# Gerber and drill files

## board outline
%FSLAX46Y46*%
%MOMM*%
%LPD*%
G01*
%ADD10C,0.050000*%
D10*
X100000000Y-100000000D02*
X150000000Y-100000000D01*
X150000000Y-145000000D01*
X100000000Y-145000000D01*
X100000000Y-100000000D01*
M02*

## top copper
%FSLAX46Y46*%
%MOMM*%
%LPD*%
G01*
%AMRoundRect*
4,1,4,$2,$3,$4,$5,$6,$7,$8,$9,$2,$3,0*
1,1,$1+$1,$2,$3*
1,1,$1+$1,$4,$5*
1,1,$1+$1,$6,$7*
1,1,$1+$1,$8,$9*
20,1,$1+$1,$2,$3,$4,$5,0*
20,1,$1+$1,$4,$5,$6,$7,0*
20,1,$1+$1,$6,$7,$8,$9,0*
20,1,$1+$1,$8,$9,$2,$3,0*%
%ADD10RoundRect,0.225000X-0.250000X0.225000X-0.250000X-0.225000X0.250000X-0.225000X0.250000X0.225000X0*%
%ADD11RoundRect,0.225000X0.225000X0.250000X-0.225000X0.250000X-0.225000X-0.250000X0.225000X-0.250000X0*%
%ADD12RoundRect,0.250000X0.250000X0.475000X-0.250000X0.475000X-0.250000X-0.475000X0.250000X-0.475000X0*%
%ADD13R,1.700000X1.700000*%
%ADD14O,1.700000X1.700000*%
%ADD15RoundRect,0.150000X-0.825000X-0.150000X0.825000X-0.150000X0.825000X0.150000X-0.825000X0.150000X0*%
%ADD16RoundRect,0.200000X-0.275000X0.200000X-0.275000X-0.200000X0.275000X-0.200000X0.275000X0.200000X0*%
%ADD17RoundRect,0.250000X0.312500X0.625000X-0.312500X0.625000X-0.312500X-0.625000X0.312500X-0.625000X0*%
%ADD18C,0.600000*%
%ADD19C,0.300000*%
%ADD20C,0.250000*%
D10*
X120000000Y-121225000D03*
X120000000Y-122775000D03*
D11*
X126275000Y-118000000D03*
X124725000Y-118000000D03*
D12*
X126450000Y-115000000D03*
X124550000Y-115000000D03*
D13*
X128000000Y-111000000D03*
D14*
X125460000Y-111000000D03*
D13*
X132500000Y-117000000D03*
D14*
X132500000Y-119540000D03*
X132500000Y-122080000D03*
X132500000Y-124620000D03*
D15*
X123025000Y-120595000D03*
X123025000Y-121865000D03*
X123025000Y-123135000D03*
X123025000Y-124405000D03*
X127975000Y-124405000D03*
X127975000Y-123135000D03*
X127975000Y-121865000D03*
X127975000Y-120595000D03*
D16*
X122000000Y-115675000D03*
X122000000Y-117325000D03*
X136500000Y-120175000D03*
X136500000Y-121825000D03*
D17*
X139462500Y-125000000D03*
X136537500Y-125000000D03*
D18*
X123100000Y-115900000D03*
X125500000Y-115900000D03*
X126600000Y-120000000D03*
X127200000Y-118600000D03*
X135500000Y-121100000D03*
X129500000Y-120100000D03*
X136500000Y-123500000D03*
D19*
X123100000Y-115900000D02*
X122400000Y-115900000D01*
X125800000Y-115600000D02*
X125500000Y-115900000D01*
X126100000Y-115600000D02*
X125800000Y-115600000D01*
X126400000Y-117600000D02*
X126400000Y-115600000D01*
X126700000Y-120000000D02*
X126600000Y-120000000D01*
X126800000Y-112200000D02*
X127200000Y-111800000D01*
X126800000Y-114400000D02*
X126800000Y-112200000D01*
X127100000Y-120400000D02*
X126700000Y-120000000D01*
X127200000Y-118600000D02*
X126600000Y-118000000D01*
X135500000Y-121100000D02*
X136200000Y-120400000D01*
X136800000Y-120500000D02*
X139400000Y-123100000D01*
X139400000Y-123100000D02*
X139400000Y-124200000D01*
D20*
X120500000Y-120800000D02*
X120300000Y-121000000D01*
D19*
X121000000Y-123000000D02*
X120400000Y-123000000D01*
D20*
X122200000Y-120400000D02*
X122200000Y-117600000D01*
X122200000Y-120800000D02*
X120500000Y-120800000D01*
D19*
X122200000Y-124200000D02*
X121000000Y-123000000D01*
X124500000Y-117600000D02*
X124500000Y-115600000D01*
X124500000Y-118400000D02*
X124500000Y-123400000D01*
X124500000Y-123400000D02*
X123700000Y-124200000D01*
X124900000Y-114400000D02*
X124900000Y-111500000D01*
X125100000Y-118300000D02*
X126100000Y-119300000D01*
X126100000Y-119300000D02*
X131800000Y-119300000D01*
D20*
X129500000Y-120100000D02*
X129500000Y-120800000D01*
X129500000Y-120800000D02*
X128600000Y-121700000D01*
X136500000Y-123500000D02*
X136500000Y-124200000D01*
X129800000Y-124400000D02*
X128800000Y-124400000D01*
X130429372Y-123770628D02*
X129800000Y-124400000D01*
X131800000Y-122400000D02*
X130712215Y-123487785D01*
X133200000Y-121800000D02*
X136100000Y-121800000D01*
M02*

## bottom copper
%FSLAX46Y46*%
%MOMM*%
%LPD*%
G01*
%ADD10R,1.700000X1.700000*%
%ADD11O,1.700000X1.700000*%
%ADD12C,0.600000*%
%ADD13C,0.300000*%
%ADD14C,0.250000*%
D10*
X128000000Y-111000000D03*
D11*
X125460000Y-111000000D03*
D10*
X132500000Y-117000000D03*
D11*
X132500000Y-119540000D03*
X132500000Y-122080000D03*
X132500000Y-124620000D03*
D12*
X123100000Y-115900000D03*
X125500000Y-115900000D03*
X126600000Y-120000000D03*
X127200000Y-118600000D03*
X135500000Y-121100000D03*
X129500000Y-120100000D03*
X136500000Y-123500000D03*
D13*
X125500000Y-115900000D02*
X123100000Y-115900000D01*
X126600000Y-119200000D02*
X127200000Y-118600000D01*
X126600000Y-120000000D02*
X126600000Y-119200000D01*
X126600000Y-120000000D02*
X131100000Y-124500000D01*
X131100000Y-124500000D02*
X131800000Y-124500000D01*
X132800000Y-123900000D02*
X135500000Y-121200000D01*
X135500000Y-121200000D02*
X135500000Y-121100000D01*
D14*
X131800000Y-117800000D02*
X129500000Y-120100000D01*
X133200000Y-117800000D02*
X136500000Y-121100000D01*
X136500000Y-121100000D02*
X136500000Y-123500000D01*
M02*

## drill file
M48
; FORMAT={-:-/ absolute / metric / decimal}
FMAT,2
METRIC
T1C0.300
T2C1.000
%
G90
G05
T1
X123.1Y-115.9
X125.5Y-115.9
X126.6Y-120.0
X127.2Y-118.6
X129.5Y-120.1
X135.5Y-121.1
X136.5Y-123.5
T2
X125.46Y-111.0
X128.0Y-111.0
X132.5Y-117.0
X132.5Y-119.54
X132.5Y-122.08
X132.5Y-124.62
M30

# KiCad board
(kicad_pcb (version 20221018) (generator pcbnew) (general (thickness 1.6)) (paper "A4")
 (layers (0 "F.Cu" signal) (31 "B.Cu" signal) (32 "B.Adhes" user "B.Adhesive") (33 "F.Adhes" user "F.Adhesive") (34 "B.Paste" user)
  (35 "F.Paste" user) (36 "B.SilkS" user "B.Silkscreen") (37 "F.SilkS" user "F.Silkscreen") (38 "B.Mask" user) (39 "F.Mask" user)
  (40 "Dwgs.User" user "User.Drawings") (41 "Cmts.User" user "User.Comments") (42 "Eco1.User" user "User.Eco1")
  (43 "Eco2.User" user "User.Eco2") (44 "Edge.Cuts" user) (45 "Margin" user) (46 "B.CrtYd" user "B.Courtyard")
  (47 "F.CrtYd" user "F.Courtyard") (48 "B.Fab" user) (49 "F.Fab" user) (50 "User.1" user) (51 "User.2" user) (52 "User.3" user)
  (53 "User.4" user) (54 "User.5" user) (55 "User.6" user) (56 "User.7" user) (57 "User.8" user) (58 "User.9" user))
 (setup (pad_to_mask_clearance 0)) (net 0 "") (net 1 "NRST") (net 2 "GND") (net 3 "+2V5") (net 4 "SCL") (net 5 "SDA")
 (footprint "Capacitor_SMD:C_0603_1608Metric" (layer "F.Cu") (at 120 122 -90)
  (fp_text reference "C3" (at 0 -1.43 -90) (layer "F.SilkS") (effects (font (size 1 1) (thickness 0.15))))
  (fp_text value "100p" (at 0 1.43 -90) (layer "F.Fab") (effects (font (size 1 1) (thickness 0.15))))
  (pad "1" smd roundrect (at -0.775 0 270) (size 0.9 0.95) (layers "F.Cu" "F.Paste" "F.Mask") (roundrect_rratio 0.25) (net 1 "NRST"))
  (pad "2" smd roundrect (at 0.775 0 270) (size 0.9 0.95) (layers "F.Cu" "F.Paste" "F.Mask") (roundrect_rratio 0.25) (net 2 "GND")))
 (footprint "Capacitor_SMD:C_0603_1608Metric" (layer "F.Cu") (at 125.5 118 180)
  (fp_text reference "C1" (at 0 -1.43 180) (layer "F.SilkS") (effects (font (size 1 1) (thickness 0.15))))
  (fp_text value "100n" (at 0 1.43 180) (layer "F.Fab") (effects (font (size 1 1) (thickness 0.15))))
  (pad "1" smd roundrect (at -0.775 0 180) (size 0.9 0.95) (layers "F.Cu" "F.Paste" "F.Mask") (roundrect_rratio 0.25) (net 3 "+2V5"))
  (pad "2" smd roundrect (at 0.775 0 180) (size 0.9 0.95) (layers "F.Cu" "F.Paste" "F.Mask") (roundrect_rratio 0.25) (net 2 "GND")))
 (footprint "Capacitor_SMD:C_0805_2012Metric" (layer "F.Cu") (at 125.5 115 180)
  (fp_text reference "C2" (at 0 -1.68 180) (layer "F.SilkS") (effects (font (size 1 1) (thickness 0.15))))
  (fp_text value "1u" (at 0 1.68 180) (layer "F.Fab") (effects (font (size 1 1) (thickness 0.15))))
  (pad "1" smd roundrect (at -0.95 0 180) (size 1 1.45) (layers "F.Cu" "F.Paste" "F.Mask") (roundrect_rratio 0.25) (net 3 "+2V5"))
  (pad "2" smd roundrect (at 0.95 0 180) (size 1 1.45) (layers "F.Cu" "F.Paste" "F.Mask") (roundrect_rratio 0.25) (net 2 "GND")))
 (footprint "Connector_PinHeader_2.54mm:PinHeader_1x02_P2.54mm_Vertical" (layer "F.Cu") (at 128 111 -90)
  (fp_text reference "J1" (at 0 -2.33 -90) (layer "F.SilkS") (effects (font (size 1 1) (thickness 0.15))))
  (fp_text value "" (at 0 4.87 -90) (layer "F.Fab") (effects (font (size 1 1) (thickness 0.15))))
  (pad "1" thru_hole rect (at 0 0 270) (size 1.7 1.7) (drill 1) (layers "*.Cu" "*.Mask") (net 3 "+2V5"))
  (pad "2" thru_hole oval (at 0 2.54 270) (size 1.7 1.7) (drill 1) (layers "*.Cu" "*.Mask") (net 2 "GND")))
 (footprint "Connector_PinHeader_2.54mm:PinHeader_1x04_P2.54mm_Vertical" (layer "F.Cu") (at 132.5 117)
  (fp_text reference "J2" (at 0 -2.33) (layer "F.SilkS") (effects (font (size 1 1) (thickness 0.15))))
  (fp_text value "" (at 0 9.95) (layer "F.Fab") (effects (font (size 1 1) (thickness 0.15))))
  (pad "1" thru_hole rect (at 0 0) (size 1.7 1.7) (drill 1) (layers "*.Cu" "*.Mask") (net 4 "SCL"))
  (pad "2" thru_hole oval (at 0 2.54) (size 1.7 1.7) (drill 1) (layers "*.Cu" "*.Mask") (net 2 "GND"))
  (pad "3" thru_hole oval (at 0 5.08) (size 1.7 1.7) (drill 1) (layers "*.Cu" "*.Mask") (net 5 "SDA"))
  (pad "4" thru_hole oval (at 0 7.62) (size 1.7 1.7) (drill 1) (layers "*.Cu" "*.Mask") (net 3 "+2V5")))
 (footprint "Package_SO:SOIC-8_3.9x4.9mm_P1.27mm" (layer "F.Cu") (at 125.5 122.5)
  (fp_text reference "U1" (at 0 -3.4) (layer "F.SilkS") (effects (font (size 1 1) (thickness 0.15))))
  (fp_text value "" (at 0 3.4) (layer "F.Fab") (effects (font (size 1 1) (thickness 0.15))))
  (pad "1" smd roundrect (at -2.475 -1.905) (size 1.95 0.6) (layers "F.Cu" "F.Paste" "F.Mask") (roundrect_rratio 0.25) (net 1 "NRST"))
  (pad "2" smd roundrect (at -2.475 -0.635) (size 1.95 0.6) (layers "F.Cu" "F.Paste" "F.Mask") (roundrect_rratio 0.25))
  (pad "3" smd roundrect (at -2.475 0.635) (size 1.95 0.6) (layers "F.Cu" "F.Paste" "F.Mask") (roundrect_rratio 0.25))
  (pad "4" smd roundrect (at -2.475 1.905) (size 1.95 0.6) (layers "F.Cu" "F.Paste" "F.Mask") (roundrect_rratio 0.25) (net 2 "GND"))
  (pad "5" smd roundrect (at 2.475 1.905) (size 1.95 0.6) (layers "F.Cu" "F.Paste" "F.Mask") (roundrect_rratio 0.25) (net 5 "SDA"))
  (pad "6" smd roundrect (at 2.475 0.635) (size 1.95 0.6) (layers "F.Cu" "F.Paste" "F.Mask") (roundrect_rratio 0.25))
  (pad "7" smd roundrect (at 2.475 -0.635) (size 1.95 0.6) (layers "F.Cu" "F.Paste" "F.Mask") (roundrect_rratio 0.25) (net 4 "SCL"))
  (pad "8" smd roundrect (at 2.475 -1.905) (size 1.95 0.6) (layers "F.Cu" "F.Paste" "F.Mask") (roundrect_rratio 0.25) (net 3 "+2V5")))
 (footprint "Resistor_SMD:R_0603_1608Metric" (layer "F.Cu") (at 122 116.5 -90)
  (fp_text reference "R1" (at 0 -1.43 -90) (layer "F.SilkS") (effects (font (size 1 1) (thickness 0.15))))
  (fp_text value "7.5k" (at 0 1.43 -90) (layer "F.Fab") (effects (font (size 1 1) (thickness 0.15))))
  (pad "1" smd roundrect (at -0.825 0 270) (size 0.8 0.95) (layers "F.Cu" "F.Paste" "F.Mask") (roundrect_rratio 0.25) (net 3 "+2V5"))
  (pad "2" smd roundrect (at 0.825 0 270) (size 0.8 0.95) (layers "F.Cu" "F.Paste" "F.Mask") (roundrect_rratio 0.25) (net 1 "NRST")))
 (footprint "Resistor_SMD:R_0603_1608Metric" (layer "F.Cu") (at 136.5 121 -90)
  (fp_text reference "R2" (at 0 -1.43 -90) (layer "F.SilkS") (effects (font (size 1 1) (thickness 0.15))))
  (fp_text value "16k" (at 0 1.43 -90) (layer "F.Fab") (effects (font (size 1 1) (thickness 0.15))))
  (pad "1" smd roundrect (at -0.825 0 270) (size 0.8 0.95) (layers "F.Cu" "F.Paste" "F.Mask") (roundrect_rratio 0.25) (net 3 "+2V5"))
  (pad "2" smd roundrect (at 0.825 0 270) (size 0.8 0.95) (layers "F.Cu" "F.Paste" "F.Mask") (roundrect_rratio 0.25) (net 5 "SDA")))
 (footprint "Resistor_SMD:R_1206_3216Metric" (layer "F.Cu") (at 138 125 180)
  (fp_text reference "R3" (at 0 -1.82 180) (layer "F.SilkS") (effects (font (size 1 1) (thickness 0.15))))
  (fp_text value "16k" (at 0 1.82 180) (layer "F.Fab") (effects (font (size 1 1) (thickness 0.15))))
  (pad "1" smd roundrect (at -1.4625 0 180) (size 1.125 1.75) (layers "F.Cu" "F.Paste" "F.Mask") (roundrect_rratio 0.222222) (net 3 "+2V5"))
  (pad "2" smd roundrect (at 1.4625 0 180) (size 1.125 1.75) (layers "F.Cu" "F.Paste" "F.Mask") (roundrect_rratio 0.222222) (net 4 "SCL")))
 (gr_rect (start 100 100) (end 150 145) (stroke (width 0.05) (type default)) (fill none) (layer "Edge.Cuts"))
 (segment (start 123.1 115.9) (end 122.4 115.9) (width 0.3) (layer "F.Cu") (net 3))
 (segment (start 125.8 115.6) (end 125.5 115.9) (width 0.3) (layer "F.Cu") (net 3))
 (segment (start 126.1 115.6) (end 125.8 115.6) (width 0.3) (layer "F.Cu") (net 3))
 (segment (start 126.4 117.6) (end 126.4 115.6) (width 0.3) (layer "F.Cu") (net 3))
 (segment (start 126.7 120) (end 126.6 120) (width 0.3) (layer "F.Cu") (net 3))
 (segment (start 126.8 112.2) (end 127.2 111.8) (width 0.3) (layer "F.Cu") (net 3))
 (segment (start 126.8 114.4) (end 126.8 112.2) (width 0.3) (layer "F.Cu") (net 3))
 (segment (start 127.1 120.4) (end 126.7 120) (width 0.3) (layer "F.Cu") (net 3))
 (segment (start 127.2 118.6) (end 126.6 118) (width 0.3) (layer "F.Cu") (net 3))
 (segment (start 135.5 121.1) (end 136.2 120.4) (width 0.3) (layer "F.Cu") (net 3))
 (segment (start 136.8 120.5) (end 139.4 123.1) (width 0.3) (layer "F.Cu") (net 3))
 (segment (start 139.4 123.1) (end 139.4 124.2) (width 0.3) (layer "F.Cu") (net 3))
 (via (at 123.1 115.9) (size 0.6) (drill 0.3) (layers "F.Cu" "B.Cu") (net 3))
 (via (at 125.5 115.9) (size 0.6) (drill 0.3) (layers "F.Cu" "B.Cu") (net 3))
 (via (at 126.6 120) (size 0.6) (drill 0.3) (layers "F.Cu" "B.Cu") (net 3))
 (via (at 127.2 118.6) (size 0.6) (drill 0.3) (layers "F.Cu" "B.Cu") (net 3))
 (via (at 135.5 121.1) (size 0.6) (drill 0.3) (layers "F.Cu" "B.Cu") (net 3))
 (segment (start 120.5 120.8) (end 120.3 121) (width 0.25) (layer "F.Cu") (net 1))
 (segment (start 121 123) (end 120.4 123) (width 0.3) (layer "F.Cu") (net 2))
 (segment (start 122.2 120.4) (end 122.2 117.6) (width 0.25) (layer "F.Cu") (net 1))
 (segment (start 122.2 120.8) (end 120.5 120.8) (width 0.25) (layer "F.Cu") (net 1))
 (segment (start 122.2 124.2) (end 121 123) (width 0.3) (layer "F.Cu") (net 2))
 (segment (start 124.5 117.6) (end 124.5 115.6) (width 0.3) (layer "F.Cu") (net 2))
 (segment (start 124.5 118.4) (end 124.5 123.4) (width 0.3) (layer "F.Cu") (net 2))
 (segment (start 124.5 123.4) (end 123.7 124.2) (width 0.3) (layer "F.Cu") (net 2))
 (segment (start 124.9 114.4) (end 124.9 111.5) (width 0.3) (layer "F.Cu") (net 2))
 (segment (start 125.1 118.3) (end 126.1 119.3) (width 0.3) (layer "F.Cu") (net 2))
 (segment (start 125.5 115.9) (end 123.1 115.9) (width 0.3) (layer "B.Cu") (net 3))
 (segment (start 126.1 119.3) (end 131.8 119.3) (width 0.3) (layer "F.Cu") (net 2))
 (segment (start 126.6 119.2) (end 127.2 118.6) (width 0.3) (layer "B.Cu") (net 3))
 (segment (start 126.6 120) (end 126.6 119.2) (width 0.3) (layer "B.Cu") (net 3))
 (segment (start 126.6 120) (end 131.1 124.5) (width 0.3) (layer "B.Cu") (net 3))
 (segment (start 129.5 120.1) (end 129.5 120.8) (width 0.25) (layer "F.Cu") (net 4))
 (segment (start 129.5 120.8) (end 128.6 121.7) (width 0.25) (layer "F.Cu") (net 4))
 (segment (start 131.1 124.5) (end 131.8 124.5) (width 0.3) (layer "B.Cu") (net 3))
 (segment (start 132.8 123.9) (end 135.5 121.2) (width 0.3) (layer "B.Cu") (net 3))
 (segment (start 135.5 121.2) (end 135.5 121.1) (width 0.3) (layer "B.Cu") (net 3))
 (segment (start 136.5 123.5) (end 136.5 124.2) (width 0.25) (layer "F.Cu") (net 4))
 (via (at 129.5 120.1) (size 0.6) (drill 0.3) (layers "F.Cu" "B.Cu") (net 4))
 (via (at 136.5 123.5) (size 0.6) (drill 0.3) (layers "F.Cu" "B.Cu") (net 4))
 (segment (start 129.8 124.4) (end 128.8 124.4) (width 0.25) (layer "F.Cu") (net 5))
 (segment (start 130.429372 123.770628) (end 129.8 124.4) (width 0.25) (layer "F.Cu") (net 5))
 (segment (start 131.8 117.8) (end 129.5 120.1) (width 0.25) (layer "B.Cu") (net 4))
 (segment (start 131.8 122.4) (end 130.712215 123.487785) (width 0.25) (layer "F.Cu") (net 5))
 (segment (start 133.2 117.8) (end 136.5 121.1) (width 0.25) (layer "B.Cu") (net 4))
 (segment (start 133.2 121.8) (end 136.1 121.8) (width 0.25) (layer "F.Cu") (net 5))
 (segment (start 136.5 121.1) (end 136.5 123.5) (width 0.25) (layer "B.Cu") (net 4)))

